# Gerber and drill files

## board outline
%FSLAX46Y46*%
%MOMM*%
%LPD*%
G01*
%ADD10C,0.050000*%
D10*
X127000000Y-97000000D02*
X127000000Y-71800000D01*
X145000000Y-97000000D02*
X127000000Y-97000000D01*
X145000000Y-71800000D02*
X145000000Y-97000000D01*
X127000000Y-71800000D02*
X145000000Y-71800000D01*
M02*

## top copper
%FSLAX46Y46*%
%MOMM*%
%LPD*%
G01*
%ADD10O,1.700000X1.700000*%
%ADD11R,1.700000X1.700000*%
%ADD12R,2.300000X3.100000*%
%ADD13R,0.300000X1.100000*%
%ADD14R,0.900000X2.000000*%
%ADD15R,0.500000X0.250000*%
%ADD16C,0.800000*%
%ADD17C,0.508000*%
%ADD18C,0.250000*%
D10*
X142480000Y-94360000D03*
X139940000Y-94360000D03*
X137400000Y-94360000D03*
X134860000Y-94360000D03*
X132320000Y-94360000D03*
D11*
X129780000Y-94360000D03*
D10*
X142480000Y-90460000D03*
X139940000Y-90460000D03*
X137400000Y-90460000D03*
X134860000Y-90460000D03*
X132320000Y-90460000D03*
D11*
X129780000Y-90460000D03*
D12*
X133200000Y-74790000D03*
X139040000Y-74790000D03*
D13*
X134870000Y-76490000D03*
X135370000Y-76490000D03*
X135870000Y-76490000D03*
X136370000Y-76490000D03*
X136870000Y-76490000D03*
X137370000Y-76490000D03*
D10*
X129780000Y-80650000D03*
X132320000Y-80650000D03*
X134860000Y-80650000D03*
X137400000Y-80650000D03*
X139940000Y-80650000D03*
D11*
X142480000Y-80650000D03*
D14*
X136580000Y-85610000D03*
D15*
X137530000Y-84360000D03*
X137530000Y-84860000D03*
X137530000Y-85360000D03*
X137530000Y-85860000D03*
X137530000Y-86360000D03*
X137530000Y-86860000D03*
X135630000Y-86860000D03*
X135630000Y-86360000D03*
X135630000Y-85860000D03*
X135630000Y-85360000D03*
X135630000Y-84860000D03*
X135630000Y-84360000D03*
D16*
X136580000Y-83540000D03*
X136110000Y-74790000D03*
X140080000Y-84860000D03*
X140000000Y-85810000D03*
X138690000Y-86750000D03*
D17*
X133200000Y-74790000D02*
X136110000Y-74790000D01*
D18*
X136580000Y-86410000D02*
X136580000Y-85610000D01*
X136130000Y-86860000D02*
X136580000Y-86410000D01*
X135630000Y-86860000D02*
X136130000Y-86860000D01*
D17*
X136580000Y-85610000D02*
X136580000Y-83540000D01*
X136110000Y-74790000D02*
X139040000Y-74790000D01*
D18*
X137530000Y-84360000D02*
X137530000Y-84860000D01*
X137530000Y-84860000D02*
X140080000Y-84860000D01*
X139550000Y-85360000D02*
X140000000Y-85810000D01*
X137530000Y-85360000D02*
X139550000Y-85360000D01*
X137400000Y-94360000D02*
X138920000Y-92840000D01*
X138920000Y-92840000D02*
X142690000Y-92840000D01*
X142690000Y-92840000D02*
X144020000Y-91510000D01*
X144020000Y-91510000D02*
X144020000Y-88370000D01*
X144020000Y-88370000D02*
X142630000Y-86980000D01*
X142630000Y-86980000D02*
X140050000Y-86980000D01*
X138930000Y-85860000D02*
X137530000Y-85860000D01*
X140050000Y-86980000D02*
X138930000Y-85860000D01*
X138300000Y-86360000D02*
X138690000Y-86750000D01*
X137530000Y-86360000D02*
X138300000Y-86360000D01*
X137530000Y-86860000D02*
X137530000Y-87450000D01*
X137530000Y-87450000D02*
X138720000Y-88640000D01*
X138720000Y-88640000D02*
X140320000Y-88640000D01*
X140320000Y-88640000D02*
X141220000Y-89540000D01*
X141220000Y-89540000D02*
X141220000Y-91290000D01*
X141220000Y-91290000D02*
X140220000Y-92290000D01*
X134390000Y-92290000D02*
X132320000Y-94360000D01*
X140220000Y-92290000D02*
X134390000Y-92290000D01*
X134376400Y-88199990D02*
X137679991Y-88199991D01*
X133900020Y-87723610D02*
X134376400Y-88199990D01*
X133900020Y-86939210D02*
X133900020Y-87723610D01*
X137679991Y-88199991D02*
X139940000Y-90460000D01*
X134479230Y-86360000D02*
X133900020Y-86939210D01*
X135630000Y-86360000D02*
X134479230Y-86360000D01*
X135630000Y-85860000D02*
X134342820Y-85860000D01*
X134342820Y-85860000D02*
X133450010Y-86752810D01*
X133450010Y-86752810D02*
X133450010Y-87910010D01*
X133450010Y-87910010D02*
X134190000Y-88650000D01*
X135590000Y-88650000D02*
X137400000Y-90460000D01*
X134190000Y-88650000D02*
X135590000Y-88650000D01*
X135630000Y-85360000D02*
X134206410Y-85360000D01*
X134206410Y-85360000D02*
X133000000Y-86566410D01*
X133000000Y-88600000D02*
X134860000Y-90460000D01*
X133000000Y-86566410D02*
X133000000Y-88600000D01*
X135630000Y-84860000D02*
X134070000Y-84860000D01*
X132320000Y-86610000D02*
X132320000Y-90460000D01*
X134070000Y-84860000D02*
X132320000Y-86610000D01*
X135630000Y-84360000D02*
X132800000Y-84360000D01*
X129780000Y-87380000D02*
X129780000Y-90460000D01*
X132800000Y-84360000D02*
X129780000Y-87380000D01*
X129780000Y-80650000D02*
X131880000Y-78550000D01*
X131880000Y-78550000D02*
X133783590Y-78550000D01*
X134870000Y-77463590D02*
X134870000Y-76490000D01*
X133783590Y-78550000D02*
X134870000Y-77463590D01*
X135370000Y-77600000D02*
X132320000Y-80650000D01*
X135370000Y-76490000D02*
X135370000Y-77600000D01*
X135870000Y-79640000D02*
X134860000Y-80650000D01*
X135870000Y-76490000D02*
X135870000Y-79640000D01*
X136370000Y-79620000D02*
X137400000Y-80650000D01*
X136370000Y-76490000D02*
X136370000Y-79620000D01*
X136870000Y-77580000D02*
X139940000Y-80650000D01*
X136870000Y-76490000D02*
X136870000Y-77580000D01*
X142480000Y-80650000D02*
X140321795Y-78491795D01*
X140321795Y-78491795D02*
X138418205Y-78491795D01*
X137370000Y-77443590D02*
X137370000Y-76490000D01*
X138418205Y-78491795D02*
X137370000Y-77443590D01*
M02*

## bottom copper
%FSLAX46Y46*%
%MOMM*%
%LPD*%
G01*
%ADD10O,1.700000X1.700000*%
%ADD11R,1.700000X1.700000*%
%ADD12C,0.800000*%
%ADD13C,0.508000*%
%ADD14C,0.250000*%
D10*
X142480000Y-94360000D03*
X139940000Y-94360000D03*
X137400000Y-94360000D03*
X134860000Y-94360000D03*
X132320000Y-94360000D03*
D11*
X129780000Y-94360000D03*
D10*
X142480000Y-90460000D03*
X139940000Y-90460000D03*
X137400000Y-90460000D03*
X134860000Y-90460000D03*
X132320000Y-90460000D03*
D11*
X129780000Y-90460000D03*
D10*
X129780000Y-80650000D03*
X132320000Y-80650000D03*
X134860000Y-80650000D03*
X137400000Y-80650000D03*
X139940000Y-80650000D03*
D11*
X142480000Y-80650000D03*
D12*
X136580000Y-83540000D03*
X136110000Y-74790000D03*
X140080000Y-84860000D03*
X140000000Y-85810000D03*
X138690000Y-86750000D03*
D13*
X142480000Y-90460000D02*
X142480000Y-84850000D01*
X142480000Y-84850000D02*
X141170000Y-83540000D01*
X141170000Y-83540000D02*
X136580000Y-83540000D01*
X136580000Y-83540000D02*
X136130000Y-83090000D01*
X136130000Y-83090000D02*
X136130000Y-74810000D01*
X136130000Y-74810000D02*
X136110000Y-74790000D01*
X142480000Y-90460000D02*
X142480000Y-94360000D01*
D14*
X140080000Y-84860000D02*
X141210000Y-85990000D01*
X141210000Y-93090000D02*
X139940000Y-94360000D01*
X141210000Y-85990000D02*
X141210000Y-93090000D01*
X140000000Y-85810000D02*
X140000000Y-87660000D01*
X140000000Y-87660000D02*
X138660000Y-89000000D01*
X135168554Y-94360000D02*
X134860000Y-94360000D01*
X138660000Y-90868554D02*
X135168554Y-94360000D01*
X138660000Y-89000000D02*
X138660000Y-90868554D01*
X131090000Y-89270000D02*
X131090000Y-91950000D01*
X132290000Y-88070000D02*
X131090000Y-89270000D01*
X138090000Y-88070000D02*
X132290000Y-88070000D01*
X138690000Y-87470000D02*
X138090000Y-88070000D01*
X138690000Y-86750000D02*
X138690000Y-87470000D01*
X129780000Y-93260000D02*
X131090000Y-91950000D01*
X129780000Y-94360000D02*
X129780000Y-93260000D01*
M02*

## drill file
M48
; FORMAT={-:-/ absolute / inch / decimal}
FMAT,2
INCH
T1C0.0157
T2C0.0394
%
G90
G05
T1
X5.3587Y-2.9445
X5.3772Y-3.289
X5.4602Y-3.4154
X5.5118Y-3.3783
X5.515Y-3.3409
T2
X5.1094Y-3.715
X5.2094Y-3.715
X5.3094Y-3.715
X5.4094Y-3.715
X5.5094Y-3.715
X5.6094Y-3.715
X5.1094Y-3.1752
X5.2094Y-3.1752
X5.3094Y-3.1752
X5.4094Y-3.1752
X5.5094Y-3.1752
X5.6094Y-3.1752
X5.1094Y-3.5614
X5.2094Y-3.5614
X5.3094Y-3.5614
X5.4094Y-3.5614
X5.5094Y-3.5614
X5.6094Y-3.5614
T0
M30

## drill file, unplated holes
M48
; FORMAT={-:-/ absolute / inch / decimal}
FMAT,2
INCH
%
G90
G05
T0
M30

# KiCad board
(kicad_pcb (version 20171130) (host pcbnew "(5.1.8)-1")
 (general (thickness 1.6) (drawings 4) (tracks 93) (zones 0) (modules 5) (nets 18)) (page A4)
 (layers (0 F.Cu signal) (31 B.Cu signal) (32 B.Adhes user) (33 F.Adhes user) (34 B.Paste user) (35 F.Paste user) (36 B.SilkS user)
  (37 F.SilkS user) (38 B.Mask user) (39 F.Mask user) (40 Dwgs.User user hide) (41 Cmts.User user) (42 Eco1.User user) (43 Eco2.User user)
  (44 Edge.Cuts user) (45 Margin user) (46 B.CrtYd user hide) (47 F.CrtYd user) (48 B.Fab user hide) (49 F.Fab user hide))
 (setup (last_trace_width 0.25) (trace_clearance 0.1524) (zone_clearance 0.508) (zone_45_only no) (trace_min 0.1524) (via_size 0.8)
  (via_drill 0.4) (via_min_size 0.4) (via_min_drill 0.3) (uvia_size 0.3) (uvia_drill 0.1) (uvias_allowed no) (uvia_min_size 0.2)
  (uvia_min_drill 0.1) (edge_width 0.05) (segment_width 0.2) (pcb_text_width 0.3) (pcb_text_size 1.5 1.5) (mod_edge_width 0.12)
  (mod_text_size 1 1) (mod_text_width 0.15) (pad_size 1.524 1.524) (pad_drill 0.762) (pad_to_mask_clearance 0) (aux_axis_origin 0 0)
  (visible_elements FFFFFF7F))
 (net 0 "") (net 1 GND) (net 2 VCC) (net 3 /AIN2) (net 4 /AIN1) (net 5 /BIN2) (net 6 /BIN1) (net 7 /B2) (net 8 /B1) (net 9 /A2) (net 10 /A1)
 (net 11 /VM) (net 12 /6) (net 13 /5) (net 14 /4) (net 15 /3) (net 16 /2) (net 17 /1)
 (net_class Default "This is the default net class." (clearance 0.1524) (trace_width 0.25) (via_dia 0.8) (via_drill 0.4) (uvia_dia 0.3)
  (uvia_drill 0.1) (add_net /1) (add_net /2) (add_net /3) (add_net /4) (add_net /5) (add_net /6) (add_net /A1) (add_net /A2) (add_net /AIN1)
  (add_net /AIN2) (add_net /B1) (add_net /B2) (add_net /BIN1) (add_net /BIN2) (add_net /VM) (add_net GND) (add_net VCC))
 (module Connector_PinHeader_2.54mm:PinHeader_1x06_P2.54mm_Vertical (layer F.Cu) (at 129.78 94.36 90)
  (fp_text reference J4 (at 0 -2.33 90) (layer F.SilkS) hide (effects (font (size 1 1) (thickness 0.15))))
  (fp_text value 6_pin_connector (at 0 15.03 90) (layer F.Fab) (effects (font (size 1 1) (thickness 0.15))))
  (pad 6 thru_hole oval (at 0 12.7 90) (size 1.7 1.7) (drill 1) (layers *.Cu *.Mask) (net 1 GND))
  (pad 5 thru_hole oval (at 0 10.16 90) (size 1.7 1.7) (drill 1) (layers *.Cu *.Mask) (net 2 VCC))
  (pad 4 thru_hole oval (at 0 7.62 90) (size 1.7 1.7) (drill 1) (layers *.Cu *.Mask) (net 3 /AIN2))
  (pad 3 thru_hole oval (at 0 5.08 90) (size 1.7 1.7) (drill 1) (layers *.Cu *.Mask) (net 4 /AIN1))
  (pad 2 thru_hole oval (at 0 2.54 90) (size 1.7 1.7) (drill 1) (layers *.Cu *.Mask) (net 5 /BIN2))
  (pad 1 thru_hole rect (at 0 0 90) (size 1.7 1.7) (drill 1) (layers *.Cu *.Mask) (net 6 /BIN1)))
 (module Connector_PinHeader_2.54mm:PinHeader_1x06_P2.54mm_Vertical (layer F.Cu) (at 129.78 90.46 90)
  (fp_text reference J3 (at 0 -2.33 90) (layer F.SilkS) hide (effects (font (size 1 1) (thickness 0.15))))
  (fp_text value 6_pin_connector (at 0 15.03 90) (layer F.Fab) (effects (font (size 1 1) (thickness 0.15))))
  (pad 6 thru_hole oval (at 0 12.7 90) (size 1.7 1.7) (drill 1) (layers *.Cu *.Mask) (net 1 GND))
  (pad 5 thru_hole oval (at 0 10.16 90) (size 1.7 1.7) (drill 1) (layers *.Cu *.Mask) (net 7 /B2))
  (pad 4 thru_hole oval (at 0 7.62 90) (size 1.7 1.7) (drill 1) (layers *.Cu *.Mask) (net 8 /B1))
  (pad 3 thru_hole oval (at 0 5.08 90) (size 1.7 1.7) (drill 1) (layers *.Cu *.Mask) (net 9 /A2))
  (pad 2 thru_hole oval (at 0 2.54 90) (size 1.7 1.7) (drill 1) (layers *.Cu *.Mask) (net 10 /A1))
  (pad 1 thru_hole rect (at 0 0 90) (size 1.7 1.7) (drill 1) (layers *.Cu *.Mask) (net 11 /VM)))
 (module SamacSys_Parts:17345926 (layer F.Cu) (at 136.12 73.99 180)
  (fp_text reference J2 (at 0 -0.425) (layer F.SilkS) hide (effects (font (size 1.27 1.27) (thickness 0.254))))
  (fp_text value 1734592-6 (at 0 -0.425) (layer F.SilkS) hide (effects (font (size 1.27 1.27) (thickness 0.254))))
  (pad MP2 smd rect (at 2.92 -0.8 180) (size 2.3 3.1) (layers F.Cu F.Paste F.Mask) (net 1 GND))
  (pad MP1 smd rect (at -2.92 -0.8 180) (size 2.3 3.1) (layers F.Cu F.Paste F.Mask) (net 1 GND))
  (pad 6 smd rect (at 1.25 -2.5 180) (size 0.3 1.1) (layers F.Cu F.Paste F.Mask) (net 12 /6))
  (pad 5 smd rect (at 0.75 -2.5 180) (size 0.3 1.1) (layers F.Cu F.Paste F.Mask) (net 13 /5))
  (pad 4 smd rect (at 0.25 -2.5 180) (size 0.3 1.1) (layers F.Cu F.Paste F.Mask) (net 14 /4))
  (pad 3 smd rect (at -0.25 -2.5 180) (size 0.3 1.1) (layers F.Cu F.Paste F.Mask) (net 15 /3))
  (pad 2 smd rect (at -0.75 -2.5 180) (size 0.3 1.1) (layers F.Cu F.Paste F.Mask) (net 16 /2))
  (pad 1 smd rect (at -1.25 -2.5 180) (size 0.3 1.1) (layers F.Cu F.Paste F.Mask) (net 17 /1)))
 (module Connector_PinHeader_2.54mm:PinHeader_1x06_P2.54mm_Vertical (layer F.Cu) (at 142.48 80.65 270)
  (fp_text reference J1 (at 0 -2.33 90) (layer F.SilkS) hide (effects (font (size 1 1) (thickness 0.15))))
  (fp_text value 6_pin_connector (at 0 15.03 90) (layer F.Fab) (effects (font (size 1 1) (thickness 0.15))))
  (pad 6 thru_hole oval (at 0 12.7 270) (size 1.7 1.7) (drill 1) (layers *.Cu *.Mask) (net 12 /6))
  (pad 5 thru_hole oval (at 0 10.16 270) (size 1.7 1.7) (drill 1) (layers *.Cu *.Mask) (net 13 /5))
  (pad 4 thru_hole oval (at 0 7.62 270) (size 1.7 1.7) (drill 1) (layers *.Cu *.Mask) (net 14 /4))
  (pad 3 thru_hole oval (at 0 5.08 270) (size 1.7 1.7) (drill 1) (layers *.Cu *.Mask) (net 15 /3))
  (pad 2 thru_hole oval (at 0 2.54 270) (size 1.7 1.7) (drill 1) (layers *.Cu *.Mask) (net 16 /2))
  (pad 1 thru_hole rect (at 0 0 270) (size 1.7 1.7) (drill 1) (layers *.Cu *.Mask) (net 17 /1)))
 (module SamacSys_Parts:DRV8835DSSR (layer F.Cu) (at 136.58 85.61)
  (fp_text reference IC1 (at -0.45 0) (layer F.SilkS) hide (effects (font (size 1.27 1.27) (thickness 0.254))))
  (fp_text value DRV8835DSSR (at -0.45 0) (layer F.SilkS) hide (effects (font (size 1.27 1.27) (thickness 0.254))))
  (pad 13 smd rect (at 0 0) (size 0.9 2) (layers F.Cu F.Paste F.Mask) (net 1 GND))
  (pad 12 smd rect (at 0.95 -1.25 90) (size 0.25 0.5) (layers F.Cu F.Paste F.Mask) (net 2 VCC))
  (pad 11 smd rect (at 0.95 -0.75 90) (size 0.25 0.5) (layers F.Cu F.Paste F.Mask) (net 2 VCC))
  (pad 10 smd rect (at 0.95 -0.25 90) (size 0.25 0.5) (layers F.Cu F.Paste F.Mask) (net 4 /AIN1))
  (pad 9 smd rect (at 0.95 0.25 90) (size 0.25 0.5) (layers F.Cu F.Paste F.Mask) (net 3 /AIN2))
  (pad 8 smd rect (at 0.95 0.75 90) (size 0.25 0.5) (layers F.Cu F.Paste F.Mask) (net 6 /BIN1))
  (pad 7 smd rect (at 0.95 1.25 90) (size 0.25 0.5) (layers F.Cu F.Paste F.Mask) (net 5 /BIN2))
  (pad 6 smd rect (at -0.95 1.25 90) (size 0.25 0.5) (layers F.Cu F.Paste F.Mask) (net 1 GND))
  (pad 5 smd rect (at -0.95 0.75 90) (size 0.25 0.5) (layers F.Cu F.Paste F.Mask) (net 7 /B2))
  (pad 4 smd rect (at -0.95 0.25 90) (size 0.25 0.5) (layers F.Cu F.Paste F.Mask) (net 8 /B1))
  (pad 3 smd rect (at -0.95 -0.25 90) (size 0.25 0.5) (layers F.Cu F.Paste F.Mask) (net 9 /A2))
  (pad 2 smd rect (at -0.95 -0.75 90) (size 0.25 0.5) (layers F.Cu F.Paste F.Mask) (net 10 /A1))
  (pad 1 smd rect (at -0.95 -1.25 90) (size 0.25 0.5) (layers F.Cu F.Paste F.Mask) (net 11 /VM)))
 (gr_line (start 127 97) (end 127 71.8) (layer Edge.Cuts) (width 0.05))
 (gr_line (start 145 97) (end 127 97) (layer Edge.Cuts) (width 0.05))
 (gr_line (start 145 71.8) (end 145 97) (layer Edge.Cuts) (width 0.05))
 (gr_line (start 127 71.8) (end 145 71.8) (layer Edge.Cuts) (width 0.05))
 (segment (start 133.2 74.79) (end 136.11 74.79) (width 0.508) (layer F.Cu) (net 1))
 (segment (start 136.58 86.41) (end 136.58 85.61) (width 0.25) (layer F.Cu) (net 1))
 (segment (start 136.13 86.86) (end 136.58 86.41) (width 0.25) (layer F.Cu) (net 1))
 (segment (start 135.63 86.86) (end 136.13 86.86) (width 0.25) (layer F.Cu) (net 1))
 (via (at 136.58 83.54) (size 0.8) (drill 0.4) (layers F.Cu B.Cu) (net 1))
 (segment (start 136.58 85.61) (end 136.58 83.54) (width 0.508) (layer F.Cu) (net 1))
 (segment (start 136.11 74.79) (end 139.04 74.79) (width 0.508) (layer F.Cu) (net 1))
 (segment (start 142.48 90.46) (end 142.48 84.85) (width 0.508) (layer B.Cu) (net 1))
 (segment (start 142.48 84.85) (end 141.17 83.54) (width 0.508) (layer B.Cu) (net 1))
 (segment (start 141.17 83.54) (end 136.58 83.54) (width 0.508) (layer B.Cu) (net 1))
 (segment (start 136.58 83.54) (end 136.13 83.09) (width 0.508) (layer B.Cu) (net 1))
 (segment (start 136.13 83.09) (end 136.13 74.81) (width 0.508) (layer B.Cu) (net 1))
 (segment (start 136.13 74.81) (end 136.11 74.79) (width 0.508) (layer B.Cu) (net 1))
 (via (at 136.11 74.79) (size 0.8) (drill 0.4) (layers F.Cu B.Cu) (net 1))
 (segment (start 142.48 90.46) (end 142.48 94.36) (width 0.508) (layer B.Cu) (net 1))
 (segment (start 137.53 84.36) (end 137.53 84.86) (width 0.25) (layer F.Cu) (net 2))
 (via (at 140.08 84.86) (size 0.8) (drill 0.4) (layers F.Cu B.Cu) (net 2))
 (segment (start 137.53 84.86) (end 140.08 84.86) (width 0.25) (layer F.Cu) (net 2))
 (segment (start 140.08 84.86) (end 141.21 85.99) (width 0.25) (layer B.Cu) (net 2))
 (segment (start 141.21 93.09) (end 139.94 94.36) (width 0.25) (layer B.Cu) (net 2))
 (segment (start 141.21 85.99) (end 141.21 93.09) (width 0.25) (layer B.Cu) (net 2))
 (via (at 140 85.81) (size 0.8) (drill 0.4) (layers F.Cu B.Cu) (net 4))
 (segment (start 139.55 85.36) (end 140 85.81) (width 0.25) (layer F.Cu) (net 4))
 (segment (start 137.53 85.36) (end 139.55 85.36) (width 0.25) (layer F.Cu) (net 4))
 (segment (start 140 85.81) (end 140 87.66) (width 0.25) (layer B.Cu) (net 4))
 (segment (start 140 87.66) (end 138.66 89) (width 0.25) (layer B.Cu) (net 4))
 (segment (start 135.168554 94.36) (end 134.86 94.36) (width 0.25) (layer B.Cu) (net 4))
 (segment (start 138.66 90.868554) (end 135.168554 94.36) (width 0.25) (layer B.Cu) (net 4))
 (segment (start 138.66 89) (end 138.66 90.868554) (width 0.25) (layer B.Cu) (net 4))
 (segment (start 137.4 94.36) (end 138.92 92.84) (width 0.25) (layer F.Cu) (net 3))
 (segment (start 138.92 92.84) (end 142.69 92.84) (width 0.25) (layer F.Cu) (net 3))
 (segment (start 142.69 92.84) (end 144.02 91.51) (width 0.25) (layer F.Cu) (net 3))
 (segment (start 144.02 91.51) (end 144.02 88.37) (width 0.25) (layer F.Cu) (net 3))
 (segment (start 144.02 88.37) (end 142.63 86.98) (width 0.25) (layer F.Cu) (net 3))
 (segment (start 142.63 86.98) (end 140.05 86.98) (width 0.25) (layer F.Cu) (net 3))
 (segment (start 138.93 85.86) (end 137.53 85.86) (width 0.25) (layer F.Cu) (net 3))
 (segment (start 140.05 86.98) (end 138.93 85.86) (width 0.25) (layer F.Cu) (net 3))
 (via (at 138.69 86.75) (size 0.8) (drill 0.4) (layers F.Cu B.Cu) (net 6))
 (segment (start 138.3 86.36) (end 138.69 86.75) (width 0.25) (layer F.Cu) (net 6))
 (segment (start 137.53 86.36) (end 138.3 86.36) (width 0.25) (layer F.Cu) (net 6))
 (segment (start 131.09 89.27) (end 131.09 91.95) (width 0.25) (layer B.Cu) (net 6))
 (segment (start 132.29 88.07) (end 131.09 89.27) (width 0.25) (layer B.Cu) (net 6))
 (segment (start 138.09 88.07) (end 132.29 88.07) (width 0.25) (layer B.Cu) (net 6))
 (segment (start 138.69 87.47) (end 138.09 88.07) (width 0.25) (layer B.Cu) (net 6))
 (segment (start 138.69 86.75) (end 138.69 87.47) (width 0.25) (layer B.Cu) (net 6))
 (segment (start 129.78 93.26) (end 131.09 91.95) (width 0.25) (layer B.Cu) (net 6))
 (segment (start 129.78 94.36) (end 129.78 93.26) (width 0.25) (layer B.Cu) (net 6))
 (segment (start 137.53 86.86) (end 137.53 87.45) (width 0.25) (layer F.Cu) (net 5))
 (segment (start 137.53 87.45) (end 138.72 88.64) (width 0.25) (layer F.Cu) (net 5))
 (segment (start 138.72 88.64) (end 140.32 88.64) (width 0.25) (layer F.Cu) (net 5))
 (segment (start 140.32 88.64) (end 141.22 89.54) (width 0.25) (layer F.Cu) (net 5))
 (segment (start 141.22 89.54) (end 141.22 91.29) (width 0.25) (layer F.Cu) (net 5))
 (segment (start 141.22 91.29) (end 140.22 92.29) (width 0.25) (layer F.Cu) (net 5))
 (segment (start 134.39 92.29) (end 132.32 94.36) (width 0.25) (layer F.Cu) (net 5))
 (segment (start 140.22 92.29) (end 134.39 92.29) (width 0.25) (layer F.Cu) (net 5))
 (segment (start 134.3764 88.19999) (end 137.679991 88.199991) (width 0.25) (layer F.Cu) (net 7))
 (segment (start 133.90002 87.72361) (end 134.3764 88.19999) (width 0.25) (layer F.Cu) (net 7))
 (segment (start 133.90002 86.93921) (end 133.90002 87.72361) (width 0.25) (layer F.Cu) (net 7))
 (segment (start 137.679991 88.199991) (end 139.94 90.46) (width 0.25) (layer F.Cu) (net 7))
 (segment (start 134.47923 86.36) (end 133.90002 86.93921) (width 0.25) (layer F.Cu) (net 7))
 (segment (start 135.63 86.36) (end 134.47923 86.36) (width 0.25) (layer F.Cu) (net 7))
 (segment (start 135.63 85.86) (end 134.34282 85.86) (width 0.25) (layer F.Cu) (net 8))
 (segment (start 134.34282 85.86) (end 133.45001 86.75281) (width 0.25) (layer F.Cu) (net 8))
 (segment (start 133.45001 86.75281) (end 133.45001 87.91001) (width 0.25) (layer F.Cu) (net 8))
 (segment (start 133.45001 87.91001) (end 134.19 88.65) (width 0.25) (layer F.Cu) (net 8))
 (segment (start 135.59 88.65) (end 137.4 90.46) (width 0.25) (layer F.Cu) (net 8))
 (segment (start 134.19 88.65) (end 135.59 88.65) (width 0.25) (layer F.Cu) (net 8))
 (segment (start 135.63 85.36) (end 134.20641 85.36) (width 0.25) (layer F.Cu) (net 9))
 (segment (start 134.20641 85.36) (end 133 86.56641) (width 0.25) (layer F.Cu) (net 9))
 (segment (start 133 88.6) (end 134.86 90.46) (width 0.25) (layer F.Cu) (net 9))
 (segment (start 133 86.56641) (end 133 88.6) (width 0.25) (layer F.Cu) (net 9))
 (segment (start 135.63 84.86) (end 134.07 84.86) (width 0.25) (layer F.Cu) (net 10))
 (segment (start 132.32 86.61) (end 132.32 90.46) (width 0.25) (layer F.Cu) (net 10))
 (segment (start 134.07 84.86) (end 132.32 86.61) (width 0.25) (layer F.Cu) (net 10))
 (segment (start 135.63 84.36) (end 132.8 84.36) (width 0.25) (layer F.Cu) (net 11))
 (segment (start 129.78 87.38) (end 129.78 90.46) (width 0.25) (layer F.Cu) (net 11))
 (segment (start 132.8 84.36) (end 129.78 87.38) (width 0.25) (layer F.Cu) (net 11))
 (segment (start 129.78 80.65) (end 131.88 78.55) (width 0.25) (layer F.Cu) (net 12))
 (segment (start 131.88 78.55) (end 133.78359 78.55) (width 0.25) (layer F.Cu) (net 12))
 (segment (start 134.87 77.46359) (end 134.87 76.49) (width 0.25) (layer F.Cu) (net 12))
 (segment (start 133.78359 78.55) (end 134.87 77.46359) (width 0.25) (layer F.Cu) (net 12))
 (segment (start 135.37 77.6) (end 132.32 80.65) (width 0.25) (layer F.Cu) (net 13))
 (segment (start 135.37 76.49) (end 135.37 77.6) (width 0.25) (layer F.Cu) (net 13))
 (segment (start 135.87 79.64) (end 134.86 80.65) (width 0.25) (layer F.Cu) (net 14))
 (segment (start 135.87 76.49) (end 135.87 79.64) (width 0.25) (layer F.Cu) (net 14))
 (segment (start 136.37 79.62) (end 137.4 80.65) (width 0.25) (layer F.Cu) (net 15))
 (segment (start 136.37 76.49) (end 136.37 79.62) (width 0.25) (layer F.Cu) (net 15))
 (segment (start 136.87 77.58) (end 139.94 80.65) (width 0.25) (layer F.Cu) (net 16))
 (segment (start 136.87 76.49) (end 136.87 77.58) (width 0.25) (layer F.Cu) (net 16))
 (segment (start 142.48 80.65) (end 140.321795 78.491795) (width 0.25) (layer F.Cu) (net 17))
 (segment (start 140.321795 78.491795) (end 138.418205 78.491795) (width 0.25) (layer F.Cu) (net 17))
 (segment (start 137.37 77.44359) (end 137.37 76.49) (width 0.25) (layer F.Cu) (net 17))
 (segment (start 138.418205 78.491795) (end 137.37 77.44359) (width 0.25) (layer F.Cu) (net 17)))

